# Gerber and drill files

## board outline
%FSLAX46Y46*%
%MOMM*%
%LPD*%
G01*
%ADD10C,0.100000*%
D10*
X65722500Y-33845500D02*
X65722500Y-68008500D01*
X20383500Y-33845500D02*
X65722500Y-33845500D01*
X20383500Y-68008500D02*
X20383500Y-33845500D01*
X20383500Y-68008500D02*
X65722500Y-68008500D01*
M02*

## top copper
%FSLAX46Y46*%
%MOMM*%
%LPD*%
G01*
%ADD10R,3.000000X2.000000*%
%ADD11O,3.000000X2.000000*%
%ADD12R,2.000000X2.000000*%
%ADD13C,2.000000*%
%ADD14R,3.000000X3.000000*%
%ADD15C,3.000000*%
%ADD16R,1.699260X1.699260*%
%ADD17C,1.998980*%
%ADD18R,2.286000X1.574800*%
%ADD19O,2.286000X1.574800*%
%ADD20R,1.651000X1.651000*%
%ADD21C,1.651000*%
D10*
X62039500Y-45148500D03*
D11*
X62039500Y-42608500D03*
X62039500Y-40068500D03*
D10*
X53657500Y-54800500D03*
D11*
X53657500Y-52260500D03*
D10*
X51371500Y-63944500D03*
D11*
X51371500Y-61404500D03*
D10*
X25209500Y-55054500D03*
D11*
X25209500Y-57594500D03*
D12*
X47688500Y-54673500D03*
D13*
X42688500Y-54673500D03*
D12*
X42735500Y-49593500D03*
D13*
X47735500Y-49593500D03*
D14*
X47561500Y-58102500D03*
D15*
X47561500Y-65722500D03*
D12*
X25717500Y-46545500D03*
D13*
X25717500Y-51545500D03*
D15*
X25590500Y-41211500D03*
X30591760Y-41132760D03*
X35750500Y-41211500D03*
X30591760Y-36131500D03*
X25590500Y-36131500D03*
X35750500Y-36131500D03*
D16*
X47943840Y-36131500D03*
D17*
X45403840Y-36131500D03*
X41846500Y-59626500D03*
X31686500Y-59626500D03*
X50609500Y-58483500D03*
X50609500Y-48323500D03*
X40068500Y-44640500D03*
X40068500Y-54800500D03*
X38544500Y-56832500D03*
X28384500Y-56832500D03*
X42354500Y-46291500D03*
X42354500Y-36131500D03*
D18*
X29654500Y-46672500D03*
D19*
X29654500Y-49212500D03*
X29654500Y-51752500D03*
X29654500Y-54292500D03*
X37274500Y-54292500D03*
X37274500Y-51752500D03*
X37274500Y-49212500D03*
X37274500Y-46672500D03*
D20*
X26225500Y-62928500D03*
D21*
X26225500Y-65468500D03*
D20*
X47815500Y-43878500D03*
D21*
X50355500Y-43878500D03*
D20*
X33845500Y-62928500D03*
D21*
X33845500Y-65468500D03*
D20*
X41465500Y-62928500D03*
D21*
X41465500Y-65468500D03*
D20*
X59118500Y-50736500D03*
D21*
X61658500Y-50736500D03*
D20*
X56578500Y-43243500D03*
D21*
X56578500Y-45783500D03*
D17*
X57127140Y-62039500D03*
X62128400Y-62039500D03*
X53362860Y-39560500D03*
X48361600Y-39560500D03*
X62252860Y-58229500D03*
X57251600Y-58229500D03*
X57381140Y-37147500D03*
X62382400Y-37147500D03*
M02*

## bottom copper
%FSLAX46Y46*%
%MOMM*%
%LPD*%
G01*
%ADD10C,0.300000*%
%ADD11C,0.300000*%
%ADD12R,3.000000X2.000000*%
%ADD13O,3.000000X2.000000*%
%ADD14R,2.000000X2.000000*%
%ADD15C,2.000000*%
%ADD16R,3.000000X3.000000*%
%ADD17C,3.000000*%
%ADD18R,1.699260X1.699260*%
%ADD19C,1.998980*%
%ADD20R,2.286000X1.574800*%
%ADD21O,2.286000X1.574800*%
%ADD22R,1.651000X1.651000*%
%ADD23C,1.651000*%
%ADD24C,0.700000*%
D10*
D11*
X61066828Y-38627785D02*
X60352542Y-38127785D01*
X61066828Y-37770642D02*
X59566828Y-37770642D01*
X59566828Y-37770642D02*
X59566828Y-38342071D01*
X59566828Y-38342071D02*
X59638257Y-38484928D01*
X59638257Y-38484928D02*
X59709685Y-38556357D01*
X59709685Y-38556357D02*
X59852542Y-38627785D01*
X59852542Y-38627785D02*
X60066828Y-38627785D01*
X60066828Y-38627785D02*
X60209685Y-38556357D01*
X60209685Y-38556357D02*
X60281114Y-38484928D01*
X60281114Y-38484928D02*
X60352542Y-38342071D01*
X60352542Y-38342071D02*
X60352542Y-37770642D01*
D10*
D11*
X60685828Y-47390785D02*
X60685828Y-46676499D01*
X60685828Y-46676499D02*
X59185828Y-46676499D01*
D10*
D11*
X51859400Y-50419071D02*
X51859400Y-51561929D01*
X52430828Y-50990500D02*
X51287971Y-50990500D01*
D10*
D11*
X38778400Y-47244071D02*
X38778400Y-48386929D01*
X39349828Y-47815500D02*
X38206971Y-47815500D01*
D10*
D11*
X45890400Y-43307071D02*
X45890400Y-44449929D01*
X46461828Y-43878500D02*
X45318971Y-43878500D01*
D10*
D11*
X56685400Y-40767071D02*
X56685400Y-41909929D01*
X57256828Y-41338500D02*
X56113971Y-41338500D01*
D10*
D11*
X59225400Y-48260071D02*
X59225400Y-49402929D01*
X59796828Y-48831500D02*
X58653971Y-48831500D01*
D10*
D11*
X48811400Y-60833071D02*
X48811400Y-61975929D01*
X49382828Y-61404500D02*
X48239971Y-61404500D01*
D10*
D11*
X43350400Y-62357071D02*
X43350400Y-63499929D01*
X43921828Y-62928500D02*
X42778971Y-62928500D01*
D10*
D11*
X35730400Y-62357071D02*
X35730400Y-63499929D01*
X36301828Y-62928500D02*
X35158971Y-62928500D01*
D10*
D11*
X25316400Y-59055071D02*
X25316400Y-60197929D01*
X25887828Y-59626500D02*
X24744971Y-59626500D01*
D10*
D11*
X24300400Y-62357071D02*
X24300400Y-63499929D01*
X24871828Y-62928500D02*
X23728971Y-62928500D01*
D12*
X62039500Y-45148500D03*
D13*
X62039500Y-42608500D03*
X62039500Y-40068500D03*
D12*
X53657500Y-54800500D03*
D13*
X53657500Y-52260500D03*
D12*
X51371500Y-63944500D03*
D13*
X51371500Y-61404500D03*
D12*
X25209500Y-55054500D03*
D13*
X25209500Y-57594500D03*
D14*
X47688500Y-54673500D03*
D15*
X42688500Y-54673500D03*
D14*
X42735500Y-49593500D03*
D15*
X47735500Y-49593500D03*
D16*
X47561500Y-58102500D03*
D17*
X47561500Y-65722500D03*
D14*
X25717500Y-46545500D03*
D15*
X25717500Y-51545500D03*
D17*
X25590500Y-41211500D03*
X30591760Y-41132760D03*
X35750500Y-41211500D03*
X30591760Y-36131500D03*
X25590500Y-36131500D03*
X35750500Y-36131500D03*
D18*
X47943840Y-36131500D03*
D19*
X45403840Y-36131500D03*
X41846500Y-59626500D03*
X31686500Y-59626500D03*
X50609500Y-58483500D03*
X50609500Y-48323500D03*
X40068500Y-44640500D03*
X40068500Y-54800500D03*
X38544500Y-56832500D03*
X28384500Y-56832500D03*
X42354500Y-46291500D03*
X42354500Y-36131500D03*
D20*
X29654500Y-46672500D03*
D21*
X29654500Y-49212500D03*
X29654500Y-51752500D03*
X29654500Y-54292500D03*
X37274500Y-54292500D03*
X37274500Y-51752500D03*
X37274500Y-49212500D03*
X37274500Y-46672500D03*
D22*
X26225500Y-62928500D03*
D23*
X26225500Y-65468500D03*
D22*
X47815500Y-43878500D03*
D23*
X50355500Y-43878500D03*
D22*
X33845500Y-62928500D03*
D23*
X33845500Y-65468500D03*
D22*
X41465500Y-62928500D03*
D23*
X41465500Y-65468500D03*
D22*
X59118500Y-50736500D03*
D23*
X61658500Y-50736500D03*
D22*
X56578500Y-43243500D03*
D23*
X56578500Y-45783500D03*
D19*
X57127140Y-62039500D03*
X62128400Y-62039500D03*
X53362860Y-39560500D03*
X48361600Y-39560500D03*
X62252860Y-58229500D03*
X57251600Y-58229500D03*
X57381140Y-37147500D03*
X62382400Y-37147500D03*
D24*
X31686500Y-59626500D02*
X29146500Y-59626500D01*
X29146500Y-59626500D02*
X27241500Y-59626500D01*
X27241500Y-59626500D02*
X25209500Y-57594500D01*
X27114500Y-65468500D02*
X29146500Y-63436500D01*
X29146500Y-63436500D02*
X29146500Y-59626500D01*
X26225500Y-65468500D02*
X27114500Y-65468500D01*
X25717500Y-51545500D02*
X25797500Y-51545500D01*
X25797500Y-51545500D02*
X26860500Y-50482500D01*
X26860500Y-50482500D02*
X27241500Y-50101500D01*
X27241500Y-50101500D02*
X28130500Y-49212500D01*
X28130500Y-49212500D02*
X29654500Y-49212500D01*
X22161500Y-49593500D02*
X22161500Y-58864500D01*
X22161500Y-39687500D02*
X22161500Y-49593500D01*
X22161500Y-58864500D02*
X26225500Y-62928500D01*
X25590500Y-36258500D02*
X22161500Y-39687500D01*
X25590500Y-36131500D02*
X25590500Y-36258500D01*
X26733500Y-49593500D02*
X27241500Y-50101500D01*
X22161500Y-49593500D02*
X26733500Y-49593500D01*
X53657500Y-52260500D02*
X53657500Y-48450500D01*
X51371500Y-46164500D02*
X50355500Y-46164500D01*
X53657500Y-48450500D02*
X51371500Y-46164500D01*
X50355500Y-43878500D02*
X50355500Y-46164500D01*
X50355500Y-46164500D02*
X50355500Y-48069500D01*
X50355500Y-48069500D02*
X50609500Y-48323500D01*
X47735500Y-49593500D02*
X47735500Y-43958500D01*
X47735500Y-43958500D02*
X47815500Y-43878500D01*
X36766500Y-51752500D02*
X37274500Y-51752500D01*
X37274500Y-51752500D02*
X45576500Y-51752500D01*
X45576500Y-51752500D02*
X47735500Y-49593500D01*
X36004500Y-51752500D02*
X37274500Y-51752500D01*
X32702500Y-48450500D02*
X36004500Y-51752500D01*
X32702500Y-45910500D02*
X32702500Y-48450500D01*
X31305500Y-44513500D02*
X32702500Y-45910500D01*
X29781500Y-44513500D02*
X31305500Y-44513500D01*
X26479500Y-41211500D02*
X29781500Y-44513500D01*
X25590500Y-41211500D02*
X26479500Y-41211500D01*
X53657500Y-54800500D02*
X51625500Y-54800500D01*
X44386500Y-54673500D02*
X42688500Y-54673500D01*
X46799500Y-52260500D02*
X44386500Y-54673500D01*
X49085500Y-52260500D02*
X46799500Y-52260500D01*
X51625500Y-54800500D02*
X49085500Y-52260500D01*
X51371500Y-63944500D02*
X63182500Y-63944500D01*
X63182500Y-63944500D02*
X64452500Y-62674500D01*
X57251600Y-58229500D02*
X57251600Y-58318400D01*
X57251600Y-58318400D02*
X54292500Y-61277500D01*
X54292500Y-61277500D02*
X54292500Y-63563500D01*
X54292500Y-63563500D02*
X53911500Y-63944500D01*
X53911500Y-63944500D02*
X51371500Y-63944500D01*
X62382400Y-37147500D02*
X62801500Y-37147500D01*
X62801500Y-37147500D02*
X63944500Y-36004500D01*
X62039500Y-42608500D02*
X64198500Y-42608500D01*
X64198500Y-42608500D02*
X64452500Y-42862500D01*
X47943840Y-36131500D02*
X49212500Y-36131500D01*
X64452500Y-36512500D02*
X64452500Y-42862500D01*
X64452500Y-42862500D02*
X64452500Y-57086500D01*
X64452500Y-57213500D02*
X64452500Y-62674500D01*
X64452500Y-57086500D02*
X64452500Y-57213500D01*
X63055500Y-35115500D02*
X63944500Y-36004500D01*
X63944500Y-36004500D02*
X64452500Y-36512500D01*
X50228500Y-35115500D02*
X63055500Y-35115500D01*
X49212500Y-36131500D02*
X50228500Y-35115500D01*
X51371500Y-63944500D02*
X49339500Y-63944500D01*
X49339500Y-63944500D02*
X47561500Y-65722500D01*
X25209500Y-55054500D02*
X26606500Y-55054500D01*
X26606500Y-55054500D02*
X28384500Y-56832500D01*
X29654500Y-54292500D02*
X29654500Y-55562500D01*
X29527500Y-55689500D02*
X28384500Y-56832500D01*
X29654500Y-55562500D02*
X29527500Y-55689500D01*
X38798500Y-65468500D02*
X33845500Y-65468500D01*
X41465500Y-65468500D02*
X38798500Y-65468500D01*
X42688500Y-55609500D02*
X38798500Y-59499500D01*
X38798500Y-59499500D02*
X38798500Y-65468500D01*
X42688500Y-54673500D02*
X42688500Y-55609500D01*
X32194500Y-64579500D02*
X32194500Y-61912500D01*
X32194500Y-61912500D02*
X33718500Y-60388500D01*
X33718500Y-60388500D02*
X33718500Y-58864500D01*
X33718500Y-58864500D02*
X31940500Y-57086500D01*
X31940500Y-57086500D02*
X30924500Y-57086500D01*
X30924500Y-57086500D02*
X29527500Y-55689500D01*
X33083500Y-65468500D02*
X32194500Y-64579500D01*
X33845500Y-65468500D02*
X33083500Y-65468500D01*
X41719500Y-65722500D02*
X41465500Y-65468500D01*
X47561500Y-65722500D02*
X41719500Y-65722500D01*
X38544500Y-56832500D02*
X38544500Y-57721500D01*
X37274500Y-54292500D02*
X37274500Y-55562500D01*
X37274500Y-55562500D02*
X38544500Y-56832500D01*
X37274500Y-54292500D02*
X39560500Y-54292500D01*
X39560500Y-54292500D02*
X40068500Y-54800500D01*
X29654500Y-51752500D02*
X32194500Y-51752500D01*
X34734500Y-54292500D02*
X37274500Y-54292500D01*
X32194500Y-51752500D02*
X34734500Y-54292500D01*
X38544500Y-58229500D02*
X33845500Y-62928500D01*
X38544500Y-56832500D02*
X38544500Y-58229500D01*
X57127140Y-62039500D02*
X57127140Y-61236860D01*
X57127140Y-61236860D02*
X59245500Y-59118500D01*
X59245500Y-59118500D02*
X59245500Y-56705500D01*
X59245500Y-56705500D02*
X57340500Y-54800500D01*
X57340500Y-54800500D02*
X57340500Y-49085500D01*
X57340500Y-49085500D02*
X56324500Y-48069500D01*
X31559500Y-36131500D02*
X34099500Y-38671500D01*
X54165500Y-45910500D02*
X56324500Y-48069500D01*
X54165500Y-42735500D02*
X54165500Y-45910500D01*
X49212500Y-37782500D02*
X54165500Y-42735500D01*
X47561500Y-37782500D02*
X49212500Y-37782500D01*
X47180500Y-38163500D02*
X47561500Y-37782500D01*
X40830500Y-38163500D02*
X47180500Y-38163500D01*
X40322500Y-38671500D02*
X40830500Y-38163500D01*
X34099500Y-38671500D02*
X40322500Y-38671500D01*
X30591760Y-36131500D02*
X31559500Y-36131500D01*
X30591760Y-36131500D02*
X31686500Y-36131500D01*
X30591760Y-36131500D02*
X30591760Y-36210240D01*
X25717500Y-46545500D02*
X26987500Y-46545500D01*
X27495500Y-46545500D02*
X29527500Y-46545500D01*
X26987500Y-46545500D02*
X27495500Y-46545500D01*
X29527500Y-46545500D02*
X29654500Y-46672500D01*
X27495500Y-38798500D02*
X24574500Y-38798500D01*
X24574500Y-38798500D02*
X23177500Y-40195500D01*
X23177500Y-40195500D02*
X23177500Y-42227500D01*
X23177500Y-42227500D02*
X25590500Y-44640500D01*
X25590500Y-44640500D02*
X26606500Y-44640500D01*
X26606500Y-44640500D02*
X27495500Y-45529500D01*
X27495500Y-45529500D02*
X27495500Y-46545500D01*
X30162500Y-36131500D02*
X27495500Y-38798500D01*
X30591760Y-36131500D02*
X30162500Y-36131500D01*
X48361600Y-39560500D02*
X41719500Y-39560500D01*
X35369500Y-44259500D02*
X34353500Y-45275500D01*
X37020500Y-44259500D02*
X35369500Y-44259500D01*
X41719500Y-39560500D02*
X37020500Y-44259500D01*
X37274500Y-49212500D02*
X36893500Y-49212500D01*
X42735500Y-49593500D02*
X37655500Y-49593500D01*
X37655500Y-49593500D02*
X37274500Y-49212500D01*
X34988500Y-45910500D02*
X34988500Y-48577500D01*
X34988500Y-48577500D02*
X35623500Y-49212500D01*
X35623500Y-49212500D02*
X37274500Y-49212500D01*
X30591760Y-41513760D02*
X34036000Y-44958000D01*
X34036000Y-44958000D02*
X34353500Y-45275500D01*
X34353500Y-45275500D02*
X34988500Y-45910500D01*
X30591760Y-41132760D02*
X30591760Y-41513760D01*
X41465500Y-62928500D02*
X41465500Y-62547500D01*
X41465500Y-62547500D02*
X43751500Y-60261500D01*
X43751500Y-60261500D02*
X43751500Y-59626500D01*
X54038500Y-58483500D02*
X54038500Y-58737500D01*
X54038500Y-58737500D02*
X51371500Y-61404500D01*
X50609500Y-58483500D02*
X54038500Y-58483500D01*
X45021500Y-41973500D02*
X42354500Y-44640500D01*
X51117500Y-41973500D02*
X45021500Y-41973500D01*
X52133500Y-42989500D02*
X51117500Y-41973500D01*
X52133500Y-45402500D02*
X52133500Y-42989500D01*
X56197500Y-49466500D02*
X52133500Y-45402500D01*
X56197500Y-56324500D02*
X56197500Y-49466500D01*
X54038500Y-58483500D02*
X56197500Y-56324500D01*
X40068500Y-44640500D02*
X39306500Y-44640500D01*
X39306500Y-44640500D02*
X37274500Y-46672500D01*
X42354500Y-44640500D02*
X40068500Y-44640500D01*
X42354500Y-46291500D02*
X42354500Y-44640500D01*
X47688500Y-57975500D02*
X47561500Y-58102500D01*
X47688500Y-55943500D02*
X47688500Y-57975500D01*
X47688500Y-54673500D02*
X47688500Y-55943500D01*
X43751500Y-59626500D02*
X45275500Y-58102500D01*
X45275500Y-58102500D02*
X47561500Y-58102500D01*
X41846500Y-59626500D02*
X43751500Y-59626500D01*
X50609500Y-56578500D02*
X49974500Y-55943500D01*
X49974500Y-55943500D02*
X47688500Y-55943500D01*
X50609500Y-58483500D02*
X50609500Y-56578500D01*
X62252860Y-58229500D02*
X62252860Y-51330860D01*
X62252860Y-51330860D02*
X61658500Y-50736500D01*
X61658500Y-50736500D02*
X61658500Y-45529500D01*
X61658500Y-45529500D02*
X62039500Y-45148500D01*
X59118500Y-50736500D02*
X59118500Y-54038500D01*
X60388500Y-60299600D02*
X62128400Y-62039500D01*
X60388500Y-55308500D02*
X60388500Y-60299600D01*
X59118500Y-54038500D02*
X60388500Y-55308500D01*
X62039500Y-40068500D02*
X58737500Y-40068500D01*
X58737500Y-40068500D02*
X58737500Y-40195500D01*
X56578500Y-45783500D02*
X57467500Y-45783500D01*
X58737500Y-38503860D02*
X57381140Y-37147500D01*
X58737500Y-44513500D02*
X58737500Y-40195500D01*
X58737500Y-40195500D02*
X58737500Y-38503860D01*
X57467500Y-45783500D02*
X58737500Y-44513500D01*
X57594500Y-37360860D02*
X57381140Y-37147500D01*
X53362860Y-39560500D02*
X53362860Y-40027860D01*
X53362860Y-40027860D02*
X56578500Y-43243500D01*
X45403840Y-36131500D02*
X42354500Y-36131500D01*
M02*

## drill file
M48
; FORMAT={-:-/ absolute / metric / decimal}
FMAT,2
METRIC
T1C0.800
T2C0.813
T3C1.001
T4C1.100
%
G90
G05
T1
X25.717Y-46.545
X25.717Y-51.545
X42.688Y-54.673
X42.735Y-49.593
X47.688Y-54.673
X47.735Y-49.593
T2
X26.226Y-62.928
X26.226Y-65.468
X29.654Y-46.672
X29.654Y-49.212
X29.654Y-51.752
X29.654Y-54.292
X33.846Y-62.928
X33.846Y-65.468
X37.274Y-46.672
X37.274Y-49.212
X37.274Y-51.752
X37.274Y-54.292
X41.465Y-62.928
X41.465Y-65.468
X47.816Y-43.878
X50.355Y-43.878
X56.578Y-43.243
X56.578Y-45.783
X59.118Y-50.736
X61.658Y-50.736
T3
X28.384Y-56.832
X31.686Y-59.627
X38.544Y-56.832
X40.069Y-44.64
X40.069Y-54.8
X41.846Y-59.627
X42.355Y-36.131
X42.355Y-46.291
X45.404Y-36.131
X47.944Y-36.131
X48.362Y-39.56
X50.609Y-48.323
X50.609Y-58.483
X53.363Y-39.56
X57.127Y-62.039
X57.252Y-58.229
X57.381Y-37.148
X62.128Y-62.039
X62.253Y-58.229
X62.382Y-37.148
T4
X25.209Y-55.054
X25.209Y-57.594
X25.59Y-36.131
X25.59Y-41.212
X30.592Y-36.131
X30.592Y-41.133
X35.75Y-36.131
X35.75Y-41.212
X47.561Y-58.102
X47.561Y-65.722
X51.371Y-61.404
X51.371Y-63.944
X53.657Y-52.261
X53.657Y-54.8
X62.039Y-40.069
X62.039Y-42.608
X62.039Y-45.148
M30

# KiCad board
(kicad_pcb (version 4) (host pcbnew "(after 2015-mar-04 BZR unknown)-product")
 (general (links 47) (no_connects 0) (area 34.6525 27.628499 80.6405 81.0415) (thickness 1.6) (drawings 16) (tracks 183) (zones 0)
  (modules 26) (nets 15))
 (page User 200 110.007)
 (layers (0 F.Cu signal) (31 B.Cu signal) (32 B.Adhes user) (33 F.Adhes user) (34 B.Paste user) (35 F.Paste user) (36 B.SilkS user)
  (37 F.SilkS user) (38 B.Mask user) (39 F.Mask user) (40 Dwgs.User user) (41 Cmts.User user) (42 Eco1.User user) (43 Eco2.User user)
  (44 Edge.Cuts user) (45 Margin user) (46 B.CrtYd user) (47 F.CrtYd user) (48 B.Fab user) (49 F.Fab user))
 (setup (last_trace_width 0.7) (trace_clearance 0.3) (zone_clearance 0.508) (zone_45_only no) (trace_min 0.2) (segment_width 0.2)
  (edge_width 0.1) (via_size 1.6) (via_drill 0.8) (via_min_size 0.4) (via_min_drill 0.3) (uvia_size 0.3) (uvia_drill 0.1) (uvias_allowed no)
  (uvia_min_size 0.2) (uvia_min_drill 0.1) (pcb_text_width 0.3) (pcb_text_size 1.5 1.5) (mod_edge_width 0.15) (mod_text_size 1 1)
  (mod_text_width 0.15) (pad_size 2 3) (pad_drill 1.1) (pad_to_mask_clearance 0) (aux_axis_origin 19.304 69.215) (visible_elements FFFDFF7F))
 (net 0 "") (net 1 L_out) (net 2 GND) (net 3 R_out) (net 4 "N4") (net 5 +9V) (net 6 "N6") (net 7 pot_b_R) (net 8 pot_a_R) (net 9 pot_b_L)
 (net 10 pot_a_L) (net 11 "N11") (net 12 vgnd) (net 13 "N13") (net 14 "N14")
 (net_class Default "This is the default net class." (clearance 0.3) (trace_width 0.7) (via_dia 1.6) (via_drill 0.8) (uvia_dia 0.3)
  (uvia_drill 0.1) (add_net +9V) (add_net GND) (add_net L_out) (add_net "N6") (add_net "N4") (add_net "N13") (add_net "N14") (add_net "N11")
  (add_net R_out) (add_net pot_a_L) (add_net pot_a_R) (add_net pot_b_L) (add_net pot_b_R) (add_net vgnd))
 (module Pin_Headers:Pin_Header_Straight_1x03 (layer F.Cu) (at 62.0395 45.1485 180)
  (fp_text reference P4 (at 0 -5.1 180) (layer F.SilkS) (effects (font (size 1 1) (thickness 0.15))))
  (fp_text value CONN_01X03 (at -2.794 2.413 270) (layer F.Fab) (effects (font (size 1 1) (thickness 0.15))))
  (pad 1 thru_hole rect (at 0 0 180) (size 3 2) (drill 1.1) (layers *.Cu *.Mask F.SilkS) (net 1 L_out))
  (pad 2 thru_hole oval (at 0 2.54 180) (size 3 2) (drill 1.1) (layers *.Cu *.Mask F.SilkS) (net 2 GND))
  (pad 3 thru_hole oval (at 0 5.08 180) (size 3 2) (drill 1.1) (layers *.Cu *.Mask F.SilkS) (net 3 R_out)))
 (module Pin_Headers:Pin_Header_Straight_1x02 (layer F.Cu) (at 53.6575 54.8005 180)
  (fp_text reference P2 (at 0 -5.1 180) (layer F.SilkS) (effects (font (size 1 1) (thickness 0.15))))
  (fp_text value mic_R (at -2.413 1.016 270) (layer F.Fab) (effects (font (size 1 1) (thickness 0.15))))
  (pad 1 thru_hole rect (at 0 0 180) (size 3 2) (drill 1.1) (layers *.Cu *.Mask F.SilkS) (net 2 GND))
  (pad 2 thru_hole oval (at 0 2.54 180) (size 3 2) (drill 1.1) (layers *.Cu *.Mask F.SilkS) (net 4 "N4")))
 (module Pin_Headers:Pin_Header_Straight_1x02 (layer F.Cu) (at 51.3715 63.9445 180)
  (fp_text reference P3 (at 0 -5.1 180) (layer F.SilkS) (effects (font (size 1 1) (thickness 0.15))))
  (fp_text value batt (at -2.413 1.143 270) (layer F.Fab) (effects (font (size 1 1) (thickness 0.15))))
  (pad 1 thru_hole rect (at 0 0 180) (size 3 2) (drill 1.1) (layers *.Cu *.Mask F.SilkS) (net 2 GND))
  (pad 2 thru_hole oval (at 0 2.54 180) (size 3 2) (drill 1.1) (layers *.Cu *.Mask F.SilkS) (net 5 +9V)))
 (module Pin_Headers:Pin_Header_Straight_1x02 (layer F.Cu) (at 25.2095 55.0545)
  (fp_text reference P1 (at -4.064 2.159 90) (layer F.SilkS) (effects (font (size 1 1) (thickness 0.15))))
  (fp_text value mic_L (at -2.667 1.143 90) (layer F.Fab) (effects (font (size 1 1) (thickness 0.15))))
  (pad 1 thru_hole rect (at 0 0) (size 3 2) (drill 1.1) (layers *.Cu *.Mask F.SilkS) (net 2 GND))
  (pad 2 thru_hole oval (at 0 2.54) (size 3 2) (drill 1.1) (layers *.Cu *.Mask F.SilkS) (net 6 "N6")))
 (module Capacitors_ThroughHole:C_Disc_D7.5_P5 (layer F.Cu) (at 47.6885 54.6735 180)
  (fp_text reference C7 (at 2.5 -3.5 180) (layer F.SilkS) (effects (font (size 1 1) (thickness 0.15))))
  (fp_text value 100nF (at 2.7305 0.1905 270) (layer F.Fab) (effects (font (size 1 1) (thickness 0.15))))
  (pad 1 thru_hole rect (at 0 0 180) (size 2 2) (drill 0.8) (layers *.Cu *.Mask F.SilkS) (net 5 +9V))
  (pad 2 thru_hole circle (at 5 0 180) (size 2 2) (drill 0.8) (layers *.Cu *.Mask F.SilkS) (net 2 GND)))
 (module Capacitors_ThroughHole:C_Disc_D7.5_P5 (layer F.Cu) (at 42.7355 49.5935)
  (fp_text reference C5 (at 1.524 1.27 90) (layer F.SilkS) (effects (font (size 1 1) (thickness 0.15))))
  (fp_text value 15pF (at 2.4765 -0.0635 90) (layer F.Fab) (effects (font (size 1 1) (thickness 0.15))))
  (pad 1 thru_hole rect (at 0 0) (size 2 2) (drill 0.8) (layers *.Cu *.Mask F.SilkS) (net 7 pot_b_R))
  (pad 2 thru_hole circle (at 5 0) (size 2 2) (drill 0.8) (layers *.Cu *.Mask F.SilkS) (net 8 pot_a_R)))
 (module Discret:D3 (layer F.Cu) (at 47.5615 61.9125 90)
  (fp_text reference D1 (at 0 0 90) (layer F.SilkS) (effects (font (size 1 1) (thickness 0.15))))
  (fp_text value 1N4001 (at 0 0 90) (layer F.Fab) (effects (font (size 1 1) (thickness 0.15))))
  (pad 1 thru_hole rect (at 3.81 0 90) (size 3 3) (drill 1.1) (layers *.Cu *.Mask F.SilkS) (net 5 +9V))
  (pad 2 thru_hole circle (at -3.81 0 90) (size 3 3) (drill 1.1) (layers *.Cu *.Mask F.SilkS) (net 2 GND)))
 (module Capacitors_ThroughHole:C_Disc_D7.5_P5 (layer F.Cu) (at 25.7175 46.5455 270)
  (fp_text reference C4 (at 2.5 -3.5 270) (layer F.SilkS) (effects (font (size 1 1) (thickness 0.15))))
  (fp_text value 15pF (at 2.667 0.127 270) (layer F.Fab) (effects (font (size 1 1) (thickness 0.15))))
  (pad 1 thru_hole rect (at 0 0 270) (size 2 2) (drill 0.8) (layers *.Cu *.Mask F.SilkS) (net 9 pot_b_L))
  (pad 2 thru_hole circle (at 5 0 270) (size 2 2) (drill 0.8) (layers *.Cu *.Mask F.SilkS) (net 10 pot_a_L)))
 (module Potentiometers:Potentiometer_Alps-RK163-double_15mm (layer F.Cu) (at 35.7505 36.1315 90)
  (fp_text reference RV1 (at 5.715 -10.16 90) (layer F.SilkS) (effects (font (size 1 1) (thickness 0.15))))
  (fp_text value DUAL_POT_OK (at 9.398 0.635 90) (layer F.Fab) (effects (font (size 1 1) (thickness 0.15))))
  (pad 23 thru_hole circle (at -5.08 -10.16 90) (size 3 3) (drill 1.1) (layers *.Cu *.Mask F.SilkS) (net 8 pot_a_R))
  (pad 22 thru_hole circle (at -5.00126 -5.15874 90) (size 3 3) (drill 1.1) (layers *.Cu *.Mask F.SilkS) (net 7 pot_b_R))
  (pad 21 thru_hole circle (at -5.08 0 90) (size 3 3) (drill 1.1) (layers *.Cu *.Mask F.SilkS))
  (pad 12 thru_hole circle (at 0 -5.15874 90) (size 3 3) (drill 1.1) (layers *.Cu *.Mask F.SilkS) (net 9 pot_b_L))
  (pad 13 thru_hole circle (at 0 -10.16 90) (size 3 3) (drill 1.1) (layers *.Cu *.Mask F.SilkS) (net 10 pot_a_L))
  (pad 11 thru_hole circle (at 0 0 90) (size 3 3) (drill 1.1) (layers *.Cu *.Mask F.SilkS)))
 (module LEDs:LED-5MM (layer F.Cu) (at 47.9425 36.1315 180)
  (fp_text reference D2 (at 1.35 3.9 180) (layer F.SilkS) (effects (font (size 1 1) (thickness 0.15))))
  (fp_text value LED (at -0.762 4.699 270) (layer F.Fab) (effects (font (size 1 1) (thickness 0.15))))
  (pad 1 thru_hole rect (at -0.00134 0 270) (size 1.69926 1.69926) (drill 1.00076) (layers *.Cu *.Mask F.SilkS) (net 2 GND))
  (pad 2 thru_hole circle (at 2.53866 0 180) (size 1.99898 1.99898) (drill 1.00076) (layers *.Cu *.Mask F.SilkS) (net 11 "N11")))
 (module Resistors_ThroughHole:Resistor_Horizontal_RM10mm (layer F.Cu) (at 36.7665 59.6265 180)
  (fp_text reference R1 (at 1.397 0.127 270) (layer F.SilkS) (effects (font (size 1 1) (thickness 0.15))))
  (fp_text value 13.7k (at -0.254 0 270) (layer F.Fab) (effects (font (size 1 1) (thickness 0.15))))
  (pad 1 thru_hole circle (at -5.08 0 180) (size 1.99898 1.99898) (drill 1.00076) (layers *.Cu *.SilkS *.Mask) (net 5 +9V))
  (pad 2 thru_hole circle (at 5.08 0 180) (size 1.99898 1.99898) (drill 1.00076) (layers *.Cu *.SilkS *.Mask) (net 6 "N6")))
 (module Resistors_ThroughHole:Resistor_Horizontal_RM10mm (layer F.Cu) (at 50.6095 53.4035 90)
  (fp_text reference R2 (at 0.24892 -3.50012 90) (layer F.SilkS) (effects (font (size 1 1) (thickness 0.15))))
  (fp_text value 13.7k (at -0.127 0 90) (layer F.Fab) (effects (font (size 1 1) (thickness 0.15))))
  (pad 1 thru_hole circle (at -5.08 0 90) (size 1.99898 1.99898) (drill 1.00076) (layers *.Cu *.SilkS *.Mask) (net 5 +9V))
  (pad 2 thru_hole circle (at 5.08 0 90) (size 1.99898 1.99898) (drill 1.00076) (layers *.Cu *.SilkS *.Mask) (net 4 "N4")))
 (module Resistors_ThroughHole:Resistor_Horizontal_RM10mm (layer F.Cu) (at 40.0685 49.7205 270)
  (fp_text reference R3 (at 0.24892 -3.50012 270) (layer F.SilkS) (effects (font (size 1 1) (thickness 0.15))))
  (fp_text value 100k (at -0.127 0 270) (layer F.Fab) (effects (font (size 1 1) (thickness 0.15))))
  (pad 1 thru_hole circle (at -5.08 0 270) (size 1.99898 1.99898) (drill 1.00076) (layers *.Cu *.SilkS *.Mask) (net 5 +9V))
  (pad 2 thru_hole circle (at 5.08 0 270) (size 1.99898 1.99898) (drill 1.00076) (layers *.Cu *.SilkS *.Mask) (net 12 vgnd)))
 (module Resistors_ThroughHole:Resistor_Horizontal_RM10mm (layer F.Cu) (at 33.4645 56.8325 180)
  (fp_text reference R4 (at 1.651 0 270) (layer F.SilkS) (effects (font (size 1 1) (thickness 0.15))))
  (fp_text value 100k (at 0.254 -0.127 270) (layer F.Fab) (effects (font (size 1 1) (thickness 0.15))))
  (pad 1 thru_hole circle (at -5.08 0 180) (size 1.99898 1.99898) (drill 1.00076) (layers *.Cu *.SilkS *.Mask) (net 12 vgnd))
  (pad 2 thru_hole circle (at 5.08 0 180) (size 1.99898 1.99898) (drill 1.00076) (layers *.Cu *.SilkS *.Mask) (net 2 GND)))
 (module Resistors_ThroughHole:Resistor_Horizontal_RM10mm (layer F.Cu) (at 42.3545 41.2115 90)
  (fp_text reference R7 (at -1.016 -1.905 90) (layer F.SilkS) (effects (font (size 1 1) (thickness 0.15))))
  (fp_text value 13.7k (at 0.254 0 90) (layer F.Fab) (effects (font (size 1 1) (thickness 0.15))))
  (pad 1 thru_hole circle (at -5.08 0 90) (size 1.99898 1.99898) (drill 1.00076) (layers *.Cu *.SilkS *.Mask) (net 5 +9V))
  (pad 2 thru_hole circle (at 5.08 0 90) (size 1.99898 1.99898) (drill 1.00076) (layers *.Cu *.SilkS *.Mask) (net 11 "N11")))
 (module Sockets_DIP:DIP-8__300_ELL (layer F.Cu) (at 33.4645 50.4825 270)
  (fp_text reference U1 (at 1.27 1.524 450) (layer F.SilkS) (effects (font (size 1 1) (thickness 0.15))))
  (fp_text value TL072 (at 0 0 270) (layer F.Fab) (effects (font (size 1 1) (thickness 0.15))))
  (pad 1 thru_hole rect (at -3.81 3.81 270) (size 1.5748 2.286) (drill 0.8128) (layers *.Cu *.Mask F.SilkS) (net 9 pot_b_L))
  (pad 2 thru_hole oval (at -1.27 3.81 270) (size 1.5748 2.286) (drill 0.8128) (layers *.Cu *.Mask F.SilkS) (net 10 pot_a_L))
  (pad 3 thru_hole oval (at 1.27 3.81 270) (size 1.5748 2.286) (drill 0.8128) (layers *.Cu *.Mask F.SilkS) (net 12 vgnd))
  (pad 4 thru_hole oval (at 3.81 3.81 270) (size 1.5748 2.286) (drill 0.8128) (layers *.Cu *.Mask F.SilkS) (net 2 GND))
  (pad 5 thru_hole oval (at 3.81 -3.81 270) (size 1.5748 2.286) (drill 0.8128) (layers *.Cu *.Mask F.SilkS) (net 12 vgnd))
  (pad 6 thru_hole oval (at 1.27 -3.81 270) (size 1.5748 2.286) (drill 0.8128) (layers *.Cu *.Mask F.SilkS) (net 8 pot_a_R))
  (pad 7 thru_hole oval (at -1.27 -3.81 270) (size 1.5748 2.286) (drill 0.8128) (layers *.Cu *.Mask F.SilkS) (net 7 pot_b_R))
  (pad 8 thru_hole oval (at -3.81 -3.81 270) (size 1.5748 2.286) (drill 0.8128) (layers *.Cu *.Mask F.SilkS) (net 5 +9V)))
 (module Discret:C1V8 (layer F.Cu) (at 26.2255 64.1985 270)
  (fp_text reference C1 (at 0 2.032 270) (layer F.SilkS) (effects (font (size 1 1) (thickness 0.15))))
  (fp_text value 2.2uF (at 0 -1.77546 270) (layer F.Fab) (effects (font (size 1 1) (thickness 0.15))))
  (pad 1 thru_hole rect (at -1.27 0 270) (size 1.651 1.651) (drill 0.8128) (layers *.Cu *.Mask F.SilkS) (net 10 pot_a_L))
  (pad 2 thru_hole circle (at 1.27 0 270) (size 1.651 1.651) (drill 0.8128) (layers *.Cu *.Mask F.SilkS) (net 6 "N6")))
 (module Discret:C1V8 (layer F.Cu) (at 49.0855 43.8785)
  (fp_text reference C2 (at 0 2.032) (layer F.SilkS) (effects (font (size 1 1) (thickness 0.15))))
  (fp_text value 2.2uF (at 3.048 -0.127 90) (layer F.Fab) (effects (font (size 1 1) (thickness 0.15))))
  (pad 1 thru_hole rect (at -1.27 0) (size 1.651 1.651) (drill 0.8128) (layers *.Cu *.Mask F.SilkS) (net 8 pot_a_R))
  (pad 2 thru_hole circle (at 1.27 0) (size 1.651 1.651) (drill 0.8128) (layers *.Cu *.Mask F.SilkS) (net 4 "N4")))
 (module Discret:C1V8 (layer F.Cu) (at 33.8455 64.1985 270)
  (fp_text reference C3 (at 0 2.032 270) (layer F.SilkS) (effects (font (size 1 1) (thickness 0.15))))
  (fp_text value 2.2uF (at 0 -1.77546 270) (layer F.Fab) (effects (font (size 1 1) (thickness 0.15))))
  (pad 1 thru_hole rect (at -1.27 0 270) (size 1.651 1.651) (drill 0.8128) (layers *.Cu *.Mask F.SilkS) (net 12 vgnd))
  (pad 2 thru_hole circle (at 1.27 0 270) (size 1.651 1.651) (drill 0.8128) (layers *.Cu *.Mask F.SilkS) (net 2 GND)))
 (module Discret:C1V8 (layer F.Cu) (at 41.4655 64.1985 270)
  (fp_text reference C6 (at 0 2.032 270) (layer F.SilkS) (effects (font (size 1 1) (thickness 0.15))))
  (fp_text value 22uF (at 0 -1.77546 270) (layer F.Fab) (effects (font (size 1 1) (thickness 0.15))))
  (pad 1 thru_hole rect (at -1.27 0 270) (size 1.651 1.651) (drill 0.8128) (layers *.Cu *.Mask F.SilkS) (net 5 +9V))
  (pad 2 thru_hole circle (at 1.27 0 270) (size 1.651 1.651) (drill 0.8128) (layers *.Cu *.Mask F.SilkS) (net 2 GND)))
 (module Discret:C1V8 (layer F.Cu) (at 60.3885 50.7365)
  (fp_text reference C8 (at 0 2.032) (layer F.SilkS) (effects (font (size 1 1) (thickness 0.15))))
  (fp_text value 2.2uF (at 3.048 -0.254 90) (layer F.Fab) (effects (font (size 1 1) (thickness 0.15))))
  (pad 1 thru_hole rect (at -1.27 0) (size 1.651 1.651) (drill 0.8128) (layers *.Cu *.Mask F.SilkS) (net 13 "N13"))
  (pad 2 thru_hole circle (at 1.27 0) (size 1.651 1.651) (drill 0.8128) (layers *.Cu *.Mask F.SilkS) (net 1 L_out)))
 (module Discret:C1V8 (layer F.Cu) (at 56.5785 44.5135 270)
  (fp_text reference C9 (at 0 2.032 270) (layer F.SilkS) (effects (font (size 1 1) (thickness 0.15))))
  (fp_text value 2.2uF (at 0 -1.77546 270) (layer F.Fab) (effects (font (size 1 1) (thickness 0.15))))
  (pad 1 thru_hole rect (at -1.27 0 270) (size 1.651 1.651) (drill 0.8128) (layers *.Cu *.Mask F.SilkS) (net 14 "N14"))
  (pad 2 thru_hole circle (at 1.27 0 270) (size 1.651 1.651) (drill 0.8128) (layers *.Cu *.Mask F.SilkS) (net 3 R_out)))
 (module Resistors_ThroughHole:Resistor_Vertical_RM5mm (layer F.Cu) (at 59.6265 62.0395)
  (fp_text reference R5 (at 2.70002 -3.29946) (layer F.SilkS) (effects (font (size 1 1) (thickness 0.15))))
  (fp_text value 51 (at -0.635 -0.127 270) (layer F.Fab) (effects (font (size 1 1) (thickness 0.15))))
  (pad 1 thru_hole circle (at -2.49936 0) (size 1.99898 1.99898) (drill 1.00076) (layers *.Cu *.SilkS *.Mask) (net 9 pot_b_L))
  (pad 2 thru_hole circle (at 2.5019 0) (size 1.99898 1.99898) (drill 1.00076) (layers *.Cu *.SilkS *.Mask) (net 13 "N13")))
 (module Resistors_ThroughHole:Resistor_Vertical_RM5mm (layer F.Cu) (at 50.8635 39.5605 180)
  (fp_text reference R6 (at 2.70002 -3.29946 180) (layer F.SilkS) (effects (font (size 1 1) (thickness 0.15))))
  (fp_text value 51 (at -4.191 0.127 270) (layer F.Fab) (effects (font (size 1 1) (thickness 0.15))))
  (pad 1 thru_hole circle (at -2.49936 0 180) (size 1.99898 1.99898) (drill 1.00076) (layers *.Cu *.SilkS *.Mask) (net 14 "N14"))
  (pad 2 thru_hole circle (at 2.5019 0 180) (size 1.99898 1.99898) (drill 1.00076) (layers *.Cu *.SilkS *.Mask) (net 7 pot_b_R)))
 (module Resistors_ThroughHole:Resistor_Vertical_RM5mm (layer F.Cu) (at 59.7535 58.2295 180)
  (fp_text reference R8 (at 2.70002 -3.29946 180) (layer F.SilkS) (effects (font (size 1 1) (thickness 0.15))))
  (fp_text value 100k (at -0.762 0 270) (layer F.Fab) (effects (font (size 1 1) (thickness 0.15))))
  (pad 1 thru_hole circle (at -2.49936 0 180) (size 1.99898 1.99898) (drill 1.00076) (layers *.Cu *.SilkS *.Mask) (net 1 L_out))
  (pad 2 thru_hole circle (at 2.5019 0 180) (size 1.99898 1.99898) (drill 1.00076) (layers *.Cu *.SilkS *.Mask) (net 2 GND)))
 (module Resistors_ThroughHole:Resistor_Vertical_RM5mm (layer F.Cu) (at 59.8805 37.1475)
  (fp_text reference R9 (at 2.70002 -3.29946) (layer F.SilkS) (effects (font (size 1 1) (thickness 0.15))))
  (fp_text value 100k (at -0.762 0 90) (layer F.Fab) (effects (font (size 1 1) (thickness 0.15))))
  (pad 1 thru_hole circle (at -2.49936 0) (size 1.99898 1.99898) (drill 1.00076) (layers *.Cu *.SilkS *.Mask) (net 3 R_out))
  (pad 2 thru_hole circle (at 2.5019 0) (size 1.99898 1.99898) (drill 1.00076) (layers *.Cu *.SilkS *.Mask) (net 2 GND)))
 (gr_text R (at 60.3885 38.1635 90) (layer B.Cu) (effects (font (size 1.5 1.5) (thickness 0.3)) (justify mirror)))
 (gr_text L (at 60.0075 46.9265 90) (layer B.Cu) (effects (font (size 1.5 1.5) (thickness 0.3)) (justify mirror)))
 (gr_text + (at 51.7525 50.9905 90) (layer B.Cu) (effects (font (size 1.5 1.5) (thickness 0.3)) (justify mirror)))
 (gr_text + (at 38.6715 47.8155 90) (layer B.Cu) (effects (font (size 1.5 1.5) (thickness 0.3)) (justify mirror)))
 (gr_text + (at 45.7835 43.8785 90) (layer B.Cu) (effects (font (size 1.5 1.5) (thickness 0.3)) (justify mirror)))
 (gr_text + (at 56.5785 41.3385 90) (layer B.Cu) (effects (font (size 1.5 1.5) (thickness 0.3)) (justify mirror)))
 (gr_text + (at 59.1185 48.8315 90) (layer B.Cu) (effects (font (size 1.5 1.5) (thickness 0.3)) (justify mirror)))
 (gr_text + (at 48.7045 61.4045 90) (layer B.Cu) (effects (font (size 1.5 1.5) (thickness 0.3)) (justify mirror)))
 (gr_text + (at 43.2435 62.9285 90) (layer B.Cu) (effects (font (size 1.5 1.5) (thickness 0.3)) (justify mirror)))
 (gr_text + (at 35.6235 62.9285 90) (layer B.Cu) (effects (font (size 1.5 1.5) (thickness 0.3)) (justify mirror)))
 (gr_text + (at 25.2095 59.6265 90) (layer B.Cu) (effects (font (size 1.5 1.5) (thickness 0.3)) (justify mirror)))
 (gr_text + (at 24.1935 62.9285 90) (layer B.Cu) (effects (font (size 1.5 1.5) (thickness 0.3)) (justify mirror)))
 (gr_line (start 65.7225 33.8455) (end 65.7225 68.0085) (angle 90) (layer Edge.Cuts) (width 0.1))
 (gr_line (start 20.3835 33.8455) (end 65.7225 33.8455) (angle 90) (layer Edge.Cuts) (width 0.1))
 (gr_line (start 20.3835 68.0085) (end 20.3835 33.8455) (angle 90) (layer Edge.Cuts) (width 0.1))
 (gr_line (start 20.3835 68.0085) (end 65.7225 68.0085) (angle 90) (layer Edge.Cuts) (width 0.1))
 (segment (start 31.6865 59.6265) (end 29.1465 59.6265) (width 0.7) (layer B.Cu) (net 6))
 (segment (start 29.1465 59.6265) (end 27.2415 59.6265) (width 0.7) (layer B.Cu) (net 6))
 (segment (start 27.2415 59.6265) (end 25.2095 57.5945) (width 0.7) (layer B.Cu) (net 6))
 (segment (start 27.1145 65.4685) (end 29.1465 63.4365) (width 0.7) (layer B.Cu) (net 6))
 (segment (start 29.1465 63.4365) (end 29.1465 59.6265) (width 0.7) (layer B.Cu) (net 6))
 (segment (start 26.2255 65.4685) (end 27.1145 65.4685) (width 0.7) (layer B.Cu) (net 6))
 (segment (start 25.7175 51.5455) (end 25.7975 51.5455) (width 0.7) (layer B.Cu) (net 10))
 (segment (start 25.7975 51.5455) (end 26.8605 50.4825) (width 0.7) (layer B.Cu) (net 10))
 (segment (start 26.8605 50.4825) (end 27.2415 50.1015) (width 0.7) (layer B.Cu) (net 10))
 (segment (start 27.2415 50.1015) (end 28.1305 49.2125) (width 0.7) (layer B.Cu) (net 10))
 (segment (start 28.1305 49.2125) (end 29.6545 49.2125) (width 0.7) (layer B.Cu) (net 10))
 (segment (start 22.1615 49.5935) (end 22.1615 58.8645) (width 0.7) (layer B.Cu) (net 10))
 (segment (start 22.1615 39.6875) (end 22.1615 49.5935) (width 0.7) (layer B.Cu) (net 10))
 (segment (start 22.1615 58.8645) (end 26.2255 62.9285) (width 0.7) (layer B.Cu) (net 10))
 (segment (start 25.5905 36.2585) (end 22.1615 39.6875) (width 0.7) (layer B.Cu) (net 10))
 (segment (start 25.5905 36.1315) (end 25.5905 36.2585) (width 0.7) (layer B.Cu) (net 10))
 (segment (start 26.7335 49.5935) (end 27.2415 50.1015) (width 0.7) (layer B.Cu) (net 10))
 (segment (start 22.1615 49.5935) (end 26.7335 49.5935) (width 0.7) (layer B.Cu) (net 10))
 (segment (start 53.6575 52.2605) (end 53.6575 48.4505) (width 0.7) (layer B.Cu) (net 4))
 (segment (start 51.3715 46.1645) (end 50.3555 46.1645) (width 0.7) (layer B.Cu) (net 4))
 (segment (start 53.6575 48.4505) (end 51.3715 46.1645) (width 0.7) (layer B.Cu) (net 4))
 (segment (start 50.3555 43.8785) (end 50.3555 46.1645) (width 0.7) (layer B.Cu) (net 4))
 (segment (start 50.3555 46.1645) (end 50.3555 48.0695) (width 0.7) (layer B.Cu) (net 4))
 (segment (start 50.3555 48.0695) (end 50.6095 48.3235) (width 0.7) (layer B.Cu) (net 4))
 (segment (start 47.7355 49.5935) (end 47.7355 43.9585) (width 0.7) (layer B.Cu) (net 8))
 (segment (start 47.7355 43.9585) (end 47.8155 43.8785) (width 0.7) (layer B.Cu) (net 8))
 (segment (start 36.7665 51.7525) (end 37.2745 51.7525) (width 0.7) (layer B.Cu) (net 8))
 (segment (start 37.2745 51.7525) (end 45.5765 51.7525) (width 0.7) (layer B.Cu) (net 8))
 (segment (start 45.5765 51.7525) (end 47.7355 49.5935) (width 0.7) (layer B.Cu) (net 8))
 (segment (start 36.0045 51.7525) (end 37.2745 51.7525) (width 0.7) (layer B.Cu) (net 8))
 (segment (start 32.7025 48.4505) (end 36.0045 51.7525) (width 0.7) (layer B.Cu) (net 8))
 (segment (start 32.7025 45.9105) (end 32.7025 48.4505) (width 0.7) (layer B.Cu) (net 8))
 (segment (start 31.3055 44.5135) (end 32.7025 45.9105) (width 0.7) (layer B.Cu) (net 8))
 (segment (start 29.7815 44.5135) (end 31.3055 44.5135) (width 0.7) (layer B.Cu) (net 8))
 (segment (start 26.4795 41.2115) (end 29.7815 44.5135) (width 0.7) (layer B.Cu) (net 8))
 (segment (start 25.5905 41.2115) (end 26.4795 41.2115) (width 0.7) (layer B.Cu) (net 8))
 (segment (start 53.6575 54.8005) (end 51.6255 54.8005) (width 0.7) (layer B.Cu) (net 2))
 (segment (start 44.3865 54.6735) (end 42.6885 54.6735) (width 0.7) (layer B.Cu) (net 2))
 (segment (start 46.7995 52.2605) (end 44.3865 54.6735) (width 0.7) (layer B.Cu) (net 2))
 (segment (start 49.0855 52.2605) (end 46.7995 52.2605) (width 0.7) (layer B.Cu) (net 2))
 (segment (start 51.6255 54.8005) (end 49.0855 52.2605) (width 0.7) (layer B.Cu) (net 2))
 (segment (start 51.3715 63.9445) (end 63.1825 63.9445) (width 0.7) (layer B.Cu) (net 2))
 (segment (start 63.1825 63.9445) (end 64.4525 62.6745) (width 0.7) (layer B.Cu) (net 2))
 (segment (start 57.2516 58.2295) (end 57.2516 58.3184) (width 0.7) (layer B.Cu) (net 2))
 (segment (start 57.2516 58.3184) (end 54.2925 61.2775) (width 0.7) (layer B.Cu) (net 2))
 (segment (start 54.2925 61.2775) (end 54.2925 63.5635) (width 0.7) (layer B.Cu) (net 2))
 (segment (start 54.2925 63.5635) (end 53.9115 63.9445) (width 0.7) (layer B.Cu) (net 2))
 (segment (start 53.9115 63.9445) (end 51.3715 63.9445) (width 0.7) (layer B.Cu) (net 2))
 (segment (start 62.3824 37.1475) (end 62.8015 37.1475) (width 0.7) (layer B.Cu) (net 2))
 (segment (start 62.8015 37.1475) (end 63.9445 36.0045) (width 0.7) (layer B.Cu) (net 2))
 (segment (start 62.0395 42.6085) (end 64.1985 42.6085) (width 0.7) (layer B.Cu) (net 2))
 (segment (start 64.1985 42.6085) (end 64.4525 42.8625) (width 0.7) (layer B.Cu) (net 2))
 (segment (start 47.94384 36.1315) (end 49.2125 36.1315) (width 0.7) (layer B.Cu) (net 2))
 (segment (start 64.4525 36.5125) (end 64.4525 42.8625) (width 0.7) (layer B.Cu) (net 2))
 (segment (start 64.4525 42.8625) (end 64.4525 57.0865) (width 0.7) (layer B.Cu) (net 2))
 (segment (start 64.4525 57.2135) (end 64.4525 62.6745) (width 0.7) (layer B.Cu) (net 2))
 (segment (start 64.4525 57.0865) (end 64.4525 57.2135) (width 0.7) (layer B.Cu) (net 2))
 (segment (start 63.0555 35.1155) (end 63.9445 36.0045) (width 0.7) (layer B.Cu) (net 2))
 (segment (start 63.9445 36.0045) (end 64.4525 36.5125) (width 0.7) (layer B.Cu) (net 2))
 (segment (start 50.2285 35.1155) (end 63.0555 35.1155) (width 0.7) (layer B.Cu) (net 2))
 (segment (start 49.2125 36.1315) (end 50.2285 35.1155) (width 0.7) (layer B.Cu) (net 2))
 (segment (start 51.3715 63.9445) (end 49.3395 63.9445) (width 0.7) (layer B.Cu) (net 2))
 (segment (start 49.3395 63.9445) (end 47.5615 65.7225) (width 0.7) (layer B.Cu) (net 2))
 (segment (start 25.2095 55.0545) (end 26.6065 55.0545) (width 0.7) (layer B.Cu) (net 2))
 (segment (start 26.6065 55.0545) (end 28.3845 56.8325) (width 0.7) (layer B.Cu) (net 2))
 (segment (start 29.6545 54.2925) (end 29.6545 55.5625) (width 0.7) (layer B.Cu) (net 2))
 (segment (start 29.5275 55.6895) (end 28.3845 56.8325) (width 0.7) (layer B.Cu) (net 2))
 (segment (start 29.6545 55.5625) (end 29.5275 55.6895) (width 0.7) (layer B.Cu) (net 2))
 (segment (start 38.7985 65.4685) (end 33.8455 65.4685) (width 0.7) (layer B.Cu) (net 2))
 (segment (start 41.4655 65.4685) (end 38.7985 65.4685) (width 0.7) (layer B.Cu) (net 2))
 (segment (start 42.6885 55.6095) (end 38.7985 59.4995) (width 0.7) (layer B.Cu) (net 2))
 (segment (start 38.7985 59.4995) (end 38.7985 65.4685) (width 0.7) (layer B.Cu) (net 2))
 (segment (start 42.6885 54.6735) (end 42.6885 55.6095) (width 0.7) (layer B.Cu) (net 2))
 (segment (start 32.1945 64.5795) (end 32.1945 61.9125) (width 0.7) (layer B.Cu) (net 2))
 (segment (start 32.1945 61.9125) (end 33.7185 60.3885) (width 0.7) (layer B.Cu) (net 2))
 (segment (start 33.7185 60.3885) (end 33.7185 58.8645) (width 0.7) (layer B.Cu) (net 2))
 (segment (start 33.7185 58.8645) (end 31.9405 57.0865) (width 0.7) (layer B.Cu) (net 2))
 (segment (start 31.9405 57.0865) (end 30.9245 57.0865) (width 0.7) (layer B.Cu) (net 2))
 (segment (start 30.9245 57.0865) (end 29.5275 55.6895) (width 0.7) (layer B.Cu) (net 2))
 (segment (start 33.0835 65.4685) (end 32.1945 64.5795) (width 0.7) (layer B.Cu) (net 2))
 (segment (start 33.8455 65.4685) (end 33.0835 65.4685) (width 0.7) (layer B.Cu) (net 2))
 (segment (start 41.7195 65.7225) (end 41.4655 65.4685) (width 0.7) (layer B.Cu) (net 2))
 (segment (start 47.5615 65.7225) (end 41.7195 65.7225) (width 0.7) (layer B.Cu) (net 2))
 (segment (start 38.5445 56.8325) (end 38.5445 57.7215) (width 0.7) (layer B.Cu) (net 12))
 (segment (start 37.2745 54.2925) (end 37.2745 55.5625) (width 0.7) (layer B.Cu) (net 12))
 (segment (start 37.2745 55.5625) (end 38.5445 56.8325) (width 0.7) (layer B.Cu) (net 12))
 (segment (start 37.2745 54.2925) (end 39.5605 54.2925) (width 0.7) (layer B.Cu) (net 12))
 (segment (start 39.5605 54.2925) (end 40.0685 54.8005) (width 0.7) (layer B.Cu) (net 12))
 (segment (start 29.6545 51.7525) (end 32.1945 51.7525) (width 0.7) (layer B.Cu) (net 12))
 (segment (start 34.7345 54.2925) (end 37.2745 54.2925) (width 0.7) (layer B.Cu) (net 12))
 (segment (start 32.1945 51.7525) (end 34.7345 54.2925) (width 0.7) (layer B.Cu) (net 12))
 (segment (start 38.5445 58.2295) (end 33.8455 62.9285) (width 0.7) (layer B.Cu) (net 12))
 (segment (start 38.5445 56.8325) (end 38.5445 58.2295) (width 0.7) (layer B.Cu) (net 12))
 (segment (start 57.12714 62.0395) (end 57.12714 61.23686) (width 0.7) (layer B.Cu) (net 9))
 (segment (start 57.12714 61.23686) (end 59.2455 59.1185) (width 0.7) (layer B.Cu) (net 9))
 (segment (start 59.2455 59.1185) (end 59.2455 56.7055) (width 0.7) (layer B.Cu) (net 9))
 (segment (start 59.2455 56.7055) (end 57.3405 54.8005) (width 0.7) (layer B.Cu) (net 9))
 (segment (start 57.3405 54.8005) (end 57.3405 49.0855) (width 0.7) (layer B.Cu) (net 9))
 (segment (start 57.3405 49.0855) (end 56.3245 48.0695) (width 0.7) (layer B.Cu) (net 9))
 (segment (start 31.5595 36.1315) (end 34.0995 38.6715) (width 0.7) (layer B.Cu) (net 9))
 (segment (start 54.1655 45.9105) (end 56.3245 48.0695) (width 0.7) (layer B.Cu) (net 9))
 (segment (start 54.1655 42.7355) (end 54.1655 45.9105) (width 0.7) (layer B.Cu) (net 9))
 (segment (start 49.2125 37.7825) (end 54.1655 42.7355) (width 0.7) (layer B.Cu) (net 9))
 (segment (start 47.5615 37.7825) (end 49.2125 37.7825) (width 0.7) (layer B.Cu) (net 9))
 (segment (start 47.1805 38.1635) (end 47.5615 37.7825) (width 0.7) (layer B.Cu) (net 9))
 (segment (start 40.8305 38.1635) (end 47.1805 38.1635) (width 0.7) (layer B.Cu) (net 9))
 (segment (start 40.3225 38.6715) (end 40.8305 38.1635) (width 0.7) (layer B.Cu) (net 9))
 (segment (start 34.0995 38.6715) (end 40.3225 38.6715) (width 0.7) (layer B.Cu) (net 9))
 (segment (start 30.59176 36.1315) (end 31.5595 36.1315) (width 0.7) (layer B.Cu) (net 9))
 (segment (start 30.59176 36.1315) (end 31.6865 36.1315) (width 0.7) (layer B.Cu) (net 9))
 (segment (start 30.59176 36.1315) (end 30.59176 36.21024) (width 0.7) (layer B.Cu) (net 9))
 (segment (start 25.7175 46.5455) (end 26.9875 46.5455) (width 0.7) (layer B.Cu) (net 9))
 (segment (start 27.4955 46.5455) (end 29.5275 46.5455) (width 0.7) (layer B.Cu) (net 9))
 (segment (start 26.9875 46.5455) (end 27.4955 46.5455) (width 0.7) (layer B.Cu) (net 9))
 (segment (start 29.5275 46.5455) (end 29.6545 46.6725) (width 0.7) (layer B.Cu) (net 9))
 (segment (start 27.4955 38.7985) (end 24.5745 38.7985) (width 0.7) (layer B.Cu) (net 9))
 (segment (start 24.5745 38.7985) (end 23.1775 40.1955) (width 0.7) (layer B.Cu) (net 9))
 (segment (start 23.1775 40.1955) (end 23.1775 42.2275) (width 0.7) (layer B.Cu) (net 9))
 (segment (start 23.1775 42.2275) (end 25.5905 44.6405) (width 0.7) (layer B.Cu) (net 9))
 (segment (start 25.5905 44.6405) (end 26.6065 44.6405) (width 0.7) (layer B.Cu) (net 9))
 (segment (start 26.6065 44.6405) (end 27.4955 45.5295) (width 0.7) (layer B.Cu) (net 9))
 (segment (start 27.4955 45.5295) (end 27.4955 46.5455) (width 0.7) (layer B.Cu) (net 9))
 (segment (start 30.1625 36.1315) (end 27.4955 38.7985) (width 0.7) (layer B.Cu) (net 9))
 (segment (start 30.59176 36.1315) (end 30.1625 36.1315) (width 0.7) (layer B.Cu) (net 9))
 (segment (start 48.3616 39.5605) (end 41.7195 39.5605) (width 0.7) (layer B.Cu) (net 7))
 (segment (start 35.3695 44.2595) (end 34.3535 45.2755) (width 0.7) (layer B.Cu) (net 7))
 (segment (start 37.0205 44.2595) (end 35.3695 44.2595) (width 0.7) (layer B.Cu) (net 7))
 (segment (start 41.7195 39.5605) (end 37.0205 44.2595) (width 0.7) (layer B.Cu) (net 7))
 (segment (start 37.2745 49.2125) (end 36.8935 49.2125) (width 0.7) (layer B.Cu) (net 7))
 (segment (start 42.7355 49.5935) (end 37.6555 49.5935) (width 0.7) (layer B.Cu) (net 7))
 (segment (start 37.6555 49.5935) (end 37.2745 49.2125) (width 0.7) (layer B.Cu) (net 7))
 (segment (start 34.9885 45.9105) (end 34.9885 48.5775) (width 0.7) (layer B.Cu) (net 7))
 (segment (start 34.9885 48.5775) (end 35.6235 49.2125) (width 0.7) (layer B.Cu) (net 7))
 (segment (start 35.6235 49.2125) (end 37.2745 49.2125) (width 0.7) (layer B.Cu) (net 7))
 (segment (start 30.59176 41.51376) (end 34.036 44.958) (width 0.7) (layer B.Cu) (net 7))
 (segment (start 34.036 44.958) (end 34.3535 45.2755) (width 0.7) (layer B.Cu) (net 7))
 (segment (start 34.3535 45.2755) (end 34.9885 45.9105) (width 0.7) (layer B.Cu) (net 7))
 (segment (start 30.59176 41.13276) (end 30.59176 41.51376) (width 0.7) (layer B.Cu) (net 7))
 (segment (start 41.4655 62.9285) (end 41.4655 62.5475) (width 0.7) (layer B.Cu) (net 5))
 (segment (start 41.4655 62.5475) (end 43.7515 60.2615) (width 0.7) (layer B.Cu) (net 5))
 (segment (start 43.7515 60.2615) (end 43.7515 59.6265) (width 0.7) (layer B.Cu) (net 5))
 (segment (start 54.0385 58.4835) (end 54.0385 58.7375) (width 0.7) (layer B.Cu) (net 5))
 (segment (start 54.0385 58.7375) (end 51.3715 61.4045) (width 0.7) (layer B.Cu) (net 5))
 (segment (start 50.6095 58.4835) (end 54.0385 58.4835) (width 0.7) (layer B.Cu) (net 5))
 (segment (start 45.0215 41.9735) (end 42.3545 44.6405) (width 0.7) (layer B.Cu) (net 5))
 (segment (start 51.1175 41.9735) (end 45.0215 41.9735) (width 0.7) (layer B.Cu) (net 5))
 (segment (start 52.1335 42.9895) (end 51.1175 41.9735) (width 0.7) (layer B.Cu) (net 5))
 (segment (start 52.1335 45.4025) (end 52.1335 42.9895) (width 0.7) (layer B.Cu) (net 5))
 (segment (start 56.1975 49.4665) (end 52.1335 45.4025) (width 0.7) (layer B.Cu) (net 5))
 (segment (start 56.1975 56.3245) (end 56.1975 49.4665) (width 0.7) (layer B.Cu) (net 5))
 (segment (start 54.0385 58.4835) (end 56.1975 56.3245) (width 0.7) (layer B.Cu) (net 5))
 (segment (start 40.0685 44.6405) (end 39.3065 44.6405) (width 0.7) (layer B.Cu) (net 5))
 (segment (start 39.3065 44.6405) (end 37.2745 46.6725) (width 0.7) (layer B.Cu) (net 5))
 (segment (start 42.3545 44.6405) (end 40.0685 44.6405) (width 0.7) (layer B.Cu) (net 5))
 (segment (start 42.3545 46.2915) (end 42.3545 44.6405) (width 0.7) (layer B.Cu) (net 5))
 (segment (start 47.6885 57.9755) (end 47.5615 58.1025) (width 0.7) (layer B.Cu) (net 5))
 (segment (start 47.6885 55.9435) (end 47.6885 57.9755) (width 0.7) (layer B.Cu) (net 5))
 (segment (start 47.6885 54.6735) (end 47.6885 55.9435) (width 0.7) (layer B.Cu) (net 5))
 (segment (start 43.7515 59.6265) (end 45.2755 58.1025) (width 0.7) (layer B.Cu) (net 5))
 (segment (start 45.2755 58.1025) (end 47.5615 58.1025) (width 0.7) (layer B.Cu) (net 5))
 (segment (start 41.8465 59.6265) (end 43.7515 59.6265) (width 0.7) (layer B.Cu) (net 5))
 (segment (start 50.6095 56.5785) (end 49.9745 55.9435) (width 0.7) (layer B.Cu) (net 5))
 (segment (start 49.9745 55.9435) (end 47.6885 55.9435) (width 0.7) (layer B.Cu) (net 5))
 (segment (start 50.6095 58.4835) (end 50.6095 56.5785) (width 0.7) (layer B.Cu) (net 5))
 (segment (start 62.25286 58.2295) (end 62.25286 51.33086) (width 0.7) (layer B.Cu) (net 1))
 (segment (start 62.25286 51.33086) (end 61.6585 50.7365) (width 0.7) (layer B.Cu) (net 1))
 (segment (start 61.6585 50.7365) (end 61.6585 45.5295) (width 0.7) (layer B.Cu) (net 1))
 (segment (start 61.6585 45.5295) (end 62.0395 45.1485) (width 0.7) (layer B.Cu) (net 1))
 (segment (start 59.1185 50.7365) (end 59.1185 54.0385) (width 0.7) (layer B.Cu) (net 13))
 (segment (start 60.3885 60.2996) (end 62.1284 62.0395) (width 0.7) (layer B.Cu) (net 13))
 (segment (start 60.3885 55.3085) (end 60.3885 60.2996) (width 0.7) (layer B.Cu) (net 13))
 (segment (start 59.1185 54.0385) (end 60.3885 55.3085) (width 0.7) (layer B.Cu) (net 13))
 (segment (start 62.0395 40.0685) (end 58.7375 40.0685) (width 0.7) (layer B.Cu) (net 3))
 (segment (start 58.7375 40.0685) (end 58.7375 40.1955) (width 0.7) (layer B.Cu) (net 3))
 (segment (start 56.5785 45.7835) (end 57.4675 45.7835) (width 0.7) (layer B.Cu) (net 3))
 (segment (start 58.7375 38.50386) (end 57.38114 37.1475) (width 0.7) (layer B.Cu) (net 3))
 (segment (start 58.7375 44.5135) (end 58.7375 40.1955) (width 0.7) (layer B.Cu) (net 3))
 (segment (start 58.7375 40.1955) (end 58.7375 38.50386) (width 0.7) (layer B.Cu) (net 3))
 (segment (start 57.4675 45.7835) (end 58.7375 44.5135) (width 0.7) (layer B.Cu) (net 3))
 (segment (start 57.5945 37.36086) (end 57.38114 37.1475) (width 0.7) (layer B.Cu) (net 3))
 (segment (start 53.36286 39.5605) (end 53.36286 40.02786) (width 0.7) (layer B.Cu) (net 14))
 (segment (start 53.36286 40.02786) (end 56.5785 43.2435) (width 0.7) (layer B.Cu) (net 14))
 (segment (start 45.40384 36.1315) (end 42.3545 36.1315) (width 0.7) (layer B.Cu) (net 11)))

